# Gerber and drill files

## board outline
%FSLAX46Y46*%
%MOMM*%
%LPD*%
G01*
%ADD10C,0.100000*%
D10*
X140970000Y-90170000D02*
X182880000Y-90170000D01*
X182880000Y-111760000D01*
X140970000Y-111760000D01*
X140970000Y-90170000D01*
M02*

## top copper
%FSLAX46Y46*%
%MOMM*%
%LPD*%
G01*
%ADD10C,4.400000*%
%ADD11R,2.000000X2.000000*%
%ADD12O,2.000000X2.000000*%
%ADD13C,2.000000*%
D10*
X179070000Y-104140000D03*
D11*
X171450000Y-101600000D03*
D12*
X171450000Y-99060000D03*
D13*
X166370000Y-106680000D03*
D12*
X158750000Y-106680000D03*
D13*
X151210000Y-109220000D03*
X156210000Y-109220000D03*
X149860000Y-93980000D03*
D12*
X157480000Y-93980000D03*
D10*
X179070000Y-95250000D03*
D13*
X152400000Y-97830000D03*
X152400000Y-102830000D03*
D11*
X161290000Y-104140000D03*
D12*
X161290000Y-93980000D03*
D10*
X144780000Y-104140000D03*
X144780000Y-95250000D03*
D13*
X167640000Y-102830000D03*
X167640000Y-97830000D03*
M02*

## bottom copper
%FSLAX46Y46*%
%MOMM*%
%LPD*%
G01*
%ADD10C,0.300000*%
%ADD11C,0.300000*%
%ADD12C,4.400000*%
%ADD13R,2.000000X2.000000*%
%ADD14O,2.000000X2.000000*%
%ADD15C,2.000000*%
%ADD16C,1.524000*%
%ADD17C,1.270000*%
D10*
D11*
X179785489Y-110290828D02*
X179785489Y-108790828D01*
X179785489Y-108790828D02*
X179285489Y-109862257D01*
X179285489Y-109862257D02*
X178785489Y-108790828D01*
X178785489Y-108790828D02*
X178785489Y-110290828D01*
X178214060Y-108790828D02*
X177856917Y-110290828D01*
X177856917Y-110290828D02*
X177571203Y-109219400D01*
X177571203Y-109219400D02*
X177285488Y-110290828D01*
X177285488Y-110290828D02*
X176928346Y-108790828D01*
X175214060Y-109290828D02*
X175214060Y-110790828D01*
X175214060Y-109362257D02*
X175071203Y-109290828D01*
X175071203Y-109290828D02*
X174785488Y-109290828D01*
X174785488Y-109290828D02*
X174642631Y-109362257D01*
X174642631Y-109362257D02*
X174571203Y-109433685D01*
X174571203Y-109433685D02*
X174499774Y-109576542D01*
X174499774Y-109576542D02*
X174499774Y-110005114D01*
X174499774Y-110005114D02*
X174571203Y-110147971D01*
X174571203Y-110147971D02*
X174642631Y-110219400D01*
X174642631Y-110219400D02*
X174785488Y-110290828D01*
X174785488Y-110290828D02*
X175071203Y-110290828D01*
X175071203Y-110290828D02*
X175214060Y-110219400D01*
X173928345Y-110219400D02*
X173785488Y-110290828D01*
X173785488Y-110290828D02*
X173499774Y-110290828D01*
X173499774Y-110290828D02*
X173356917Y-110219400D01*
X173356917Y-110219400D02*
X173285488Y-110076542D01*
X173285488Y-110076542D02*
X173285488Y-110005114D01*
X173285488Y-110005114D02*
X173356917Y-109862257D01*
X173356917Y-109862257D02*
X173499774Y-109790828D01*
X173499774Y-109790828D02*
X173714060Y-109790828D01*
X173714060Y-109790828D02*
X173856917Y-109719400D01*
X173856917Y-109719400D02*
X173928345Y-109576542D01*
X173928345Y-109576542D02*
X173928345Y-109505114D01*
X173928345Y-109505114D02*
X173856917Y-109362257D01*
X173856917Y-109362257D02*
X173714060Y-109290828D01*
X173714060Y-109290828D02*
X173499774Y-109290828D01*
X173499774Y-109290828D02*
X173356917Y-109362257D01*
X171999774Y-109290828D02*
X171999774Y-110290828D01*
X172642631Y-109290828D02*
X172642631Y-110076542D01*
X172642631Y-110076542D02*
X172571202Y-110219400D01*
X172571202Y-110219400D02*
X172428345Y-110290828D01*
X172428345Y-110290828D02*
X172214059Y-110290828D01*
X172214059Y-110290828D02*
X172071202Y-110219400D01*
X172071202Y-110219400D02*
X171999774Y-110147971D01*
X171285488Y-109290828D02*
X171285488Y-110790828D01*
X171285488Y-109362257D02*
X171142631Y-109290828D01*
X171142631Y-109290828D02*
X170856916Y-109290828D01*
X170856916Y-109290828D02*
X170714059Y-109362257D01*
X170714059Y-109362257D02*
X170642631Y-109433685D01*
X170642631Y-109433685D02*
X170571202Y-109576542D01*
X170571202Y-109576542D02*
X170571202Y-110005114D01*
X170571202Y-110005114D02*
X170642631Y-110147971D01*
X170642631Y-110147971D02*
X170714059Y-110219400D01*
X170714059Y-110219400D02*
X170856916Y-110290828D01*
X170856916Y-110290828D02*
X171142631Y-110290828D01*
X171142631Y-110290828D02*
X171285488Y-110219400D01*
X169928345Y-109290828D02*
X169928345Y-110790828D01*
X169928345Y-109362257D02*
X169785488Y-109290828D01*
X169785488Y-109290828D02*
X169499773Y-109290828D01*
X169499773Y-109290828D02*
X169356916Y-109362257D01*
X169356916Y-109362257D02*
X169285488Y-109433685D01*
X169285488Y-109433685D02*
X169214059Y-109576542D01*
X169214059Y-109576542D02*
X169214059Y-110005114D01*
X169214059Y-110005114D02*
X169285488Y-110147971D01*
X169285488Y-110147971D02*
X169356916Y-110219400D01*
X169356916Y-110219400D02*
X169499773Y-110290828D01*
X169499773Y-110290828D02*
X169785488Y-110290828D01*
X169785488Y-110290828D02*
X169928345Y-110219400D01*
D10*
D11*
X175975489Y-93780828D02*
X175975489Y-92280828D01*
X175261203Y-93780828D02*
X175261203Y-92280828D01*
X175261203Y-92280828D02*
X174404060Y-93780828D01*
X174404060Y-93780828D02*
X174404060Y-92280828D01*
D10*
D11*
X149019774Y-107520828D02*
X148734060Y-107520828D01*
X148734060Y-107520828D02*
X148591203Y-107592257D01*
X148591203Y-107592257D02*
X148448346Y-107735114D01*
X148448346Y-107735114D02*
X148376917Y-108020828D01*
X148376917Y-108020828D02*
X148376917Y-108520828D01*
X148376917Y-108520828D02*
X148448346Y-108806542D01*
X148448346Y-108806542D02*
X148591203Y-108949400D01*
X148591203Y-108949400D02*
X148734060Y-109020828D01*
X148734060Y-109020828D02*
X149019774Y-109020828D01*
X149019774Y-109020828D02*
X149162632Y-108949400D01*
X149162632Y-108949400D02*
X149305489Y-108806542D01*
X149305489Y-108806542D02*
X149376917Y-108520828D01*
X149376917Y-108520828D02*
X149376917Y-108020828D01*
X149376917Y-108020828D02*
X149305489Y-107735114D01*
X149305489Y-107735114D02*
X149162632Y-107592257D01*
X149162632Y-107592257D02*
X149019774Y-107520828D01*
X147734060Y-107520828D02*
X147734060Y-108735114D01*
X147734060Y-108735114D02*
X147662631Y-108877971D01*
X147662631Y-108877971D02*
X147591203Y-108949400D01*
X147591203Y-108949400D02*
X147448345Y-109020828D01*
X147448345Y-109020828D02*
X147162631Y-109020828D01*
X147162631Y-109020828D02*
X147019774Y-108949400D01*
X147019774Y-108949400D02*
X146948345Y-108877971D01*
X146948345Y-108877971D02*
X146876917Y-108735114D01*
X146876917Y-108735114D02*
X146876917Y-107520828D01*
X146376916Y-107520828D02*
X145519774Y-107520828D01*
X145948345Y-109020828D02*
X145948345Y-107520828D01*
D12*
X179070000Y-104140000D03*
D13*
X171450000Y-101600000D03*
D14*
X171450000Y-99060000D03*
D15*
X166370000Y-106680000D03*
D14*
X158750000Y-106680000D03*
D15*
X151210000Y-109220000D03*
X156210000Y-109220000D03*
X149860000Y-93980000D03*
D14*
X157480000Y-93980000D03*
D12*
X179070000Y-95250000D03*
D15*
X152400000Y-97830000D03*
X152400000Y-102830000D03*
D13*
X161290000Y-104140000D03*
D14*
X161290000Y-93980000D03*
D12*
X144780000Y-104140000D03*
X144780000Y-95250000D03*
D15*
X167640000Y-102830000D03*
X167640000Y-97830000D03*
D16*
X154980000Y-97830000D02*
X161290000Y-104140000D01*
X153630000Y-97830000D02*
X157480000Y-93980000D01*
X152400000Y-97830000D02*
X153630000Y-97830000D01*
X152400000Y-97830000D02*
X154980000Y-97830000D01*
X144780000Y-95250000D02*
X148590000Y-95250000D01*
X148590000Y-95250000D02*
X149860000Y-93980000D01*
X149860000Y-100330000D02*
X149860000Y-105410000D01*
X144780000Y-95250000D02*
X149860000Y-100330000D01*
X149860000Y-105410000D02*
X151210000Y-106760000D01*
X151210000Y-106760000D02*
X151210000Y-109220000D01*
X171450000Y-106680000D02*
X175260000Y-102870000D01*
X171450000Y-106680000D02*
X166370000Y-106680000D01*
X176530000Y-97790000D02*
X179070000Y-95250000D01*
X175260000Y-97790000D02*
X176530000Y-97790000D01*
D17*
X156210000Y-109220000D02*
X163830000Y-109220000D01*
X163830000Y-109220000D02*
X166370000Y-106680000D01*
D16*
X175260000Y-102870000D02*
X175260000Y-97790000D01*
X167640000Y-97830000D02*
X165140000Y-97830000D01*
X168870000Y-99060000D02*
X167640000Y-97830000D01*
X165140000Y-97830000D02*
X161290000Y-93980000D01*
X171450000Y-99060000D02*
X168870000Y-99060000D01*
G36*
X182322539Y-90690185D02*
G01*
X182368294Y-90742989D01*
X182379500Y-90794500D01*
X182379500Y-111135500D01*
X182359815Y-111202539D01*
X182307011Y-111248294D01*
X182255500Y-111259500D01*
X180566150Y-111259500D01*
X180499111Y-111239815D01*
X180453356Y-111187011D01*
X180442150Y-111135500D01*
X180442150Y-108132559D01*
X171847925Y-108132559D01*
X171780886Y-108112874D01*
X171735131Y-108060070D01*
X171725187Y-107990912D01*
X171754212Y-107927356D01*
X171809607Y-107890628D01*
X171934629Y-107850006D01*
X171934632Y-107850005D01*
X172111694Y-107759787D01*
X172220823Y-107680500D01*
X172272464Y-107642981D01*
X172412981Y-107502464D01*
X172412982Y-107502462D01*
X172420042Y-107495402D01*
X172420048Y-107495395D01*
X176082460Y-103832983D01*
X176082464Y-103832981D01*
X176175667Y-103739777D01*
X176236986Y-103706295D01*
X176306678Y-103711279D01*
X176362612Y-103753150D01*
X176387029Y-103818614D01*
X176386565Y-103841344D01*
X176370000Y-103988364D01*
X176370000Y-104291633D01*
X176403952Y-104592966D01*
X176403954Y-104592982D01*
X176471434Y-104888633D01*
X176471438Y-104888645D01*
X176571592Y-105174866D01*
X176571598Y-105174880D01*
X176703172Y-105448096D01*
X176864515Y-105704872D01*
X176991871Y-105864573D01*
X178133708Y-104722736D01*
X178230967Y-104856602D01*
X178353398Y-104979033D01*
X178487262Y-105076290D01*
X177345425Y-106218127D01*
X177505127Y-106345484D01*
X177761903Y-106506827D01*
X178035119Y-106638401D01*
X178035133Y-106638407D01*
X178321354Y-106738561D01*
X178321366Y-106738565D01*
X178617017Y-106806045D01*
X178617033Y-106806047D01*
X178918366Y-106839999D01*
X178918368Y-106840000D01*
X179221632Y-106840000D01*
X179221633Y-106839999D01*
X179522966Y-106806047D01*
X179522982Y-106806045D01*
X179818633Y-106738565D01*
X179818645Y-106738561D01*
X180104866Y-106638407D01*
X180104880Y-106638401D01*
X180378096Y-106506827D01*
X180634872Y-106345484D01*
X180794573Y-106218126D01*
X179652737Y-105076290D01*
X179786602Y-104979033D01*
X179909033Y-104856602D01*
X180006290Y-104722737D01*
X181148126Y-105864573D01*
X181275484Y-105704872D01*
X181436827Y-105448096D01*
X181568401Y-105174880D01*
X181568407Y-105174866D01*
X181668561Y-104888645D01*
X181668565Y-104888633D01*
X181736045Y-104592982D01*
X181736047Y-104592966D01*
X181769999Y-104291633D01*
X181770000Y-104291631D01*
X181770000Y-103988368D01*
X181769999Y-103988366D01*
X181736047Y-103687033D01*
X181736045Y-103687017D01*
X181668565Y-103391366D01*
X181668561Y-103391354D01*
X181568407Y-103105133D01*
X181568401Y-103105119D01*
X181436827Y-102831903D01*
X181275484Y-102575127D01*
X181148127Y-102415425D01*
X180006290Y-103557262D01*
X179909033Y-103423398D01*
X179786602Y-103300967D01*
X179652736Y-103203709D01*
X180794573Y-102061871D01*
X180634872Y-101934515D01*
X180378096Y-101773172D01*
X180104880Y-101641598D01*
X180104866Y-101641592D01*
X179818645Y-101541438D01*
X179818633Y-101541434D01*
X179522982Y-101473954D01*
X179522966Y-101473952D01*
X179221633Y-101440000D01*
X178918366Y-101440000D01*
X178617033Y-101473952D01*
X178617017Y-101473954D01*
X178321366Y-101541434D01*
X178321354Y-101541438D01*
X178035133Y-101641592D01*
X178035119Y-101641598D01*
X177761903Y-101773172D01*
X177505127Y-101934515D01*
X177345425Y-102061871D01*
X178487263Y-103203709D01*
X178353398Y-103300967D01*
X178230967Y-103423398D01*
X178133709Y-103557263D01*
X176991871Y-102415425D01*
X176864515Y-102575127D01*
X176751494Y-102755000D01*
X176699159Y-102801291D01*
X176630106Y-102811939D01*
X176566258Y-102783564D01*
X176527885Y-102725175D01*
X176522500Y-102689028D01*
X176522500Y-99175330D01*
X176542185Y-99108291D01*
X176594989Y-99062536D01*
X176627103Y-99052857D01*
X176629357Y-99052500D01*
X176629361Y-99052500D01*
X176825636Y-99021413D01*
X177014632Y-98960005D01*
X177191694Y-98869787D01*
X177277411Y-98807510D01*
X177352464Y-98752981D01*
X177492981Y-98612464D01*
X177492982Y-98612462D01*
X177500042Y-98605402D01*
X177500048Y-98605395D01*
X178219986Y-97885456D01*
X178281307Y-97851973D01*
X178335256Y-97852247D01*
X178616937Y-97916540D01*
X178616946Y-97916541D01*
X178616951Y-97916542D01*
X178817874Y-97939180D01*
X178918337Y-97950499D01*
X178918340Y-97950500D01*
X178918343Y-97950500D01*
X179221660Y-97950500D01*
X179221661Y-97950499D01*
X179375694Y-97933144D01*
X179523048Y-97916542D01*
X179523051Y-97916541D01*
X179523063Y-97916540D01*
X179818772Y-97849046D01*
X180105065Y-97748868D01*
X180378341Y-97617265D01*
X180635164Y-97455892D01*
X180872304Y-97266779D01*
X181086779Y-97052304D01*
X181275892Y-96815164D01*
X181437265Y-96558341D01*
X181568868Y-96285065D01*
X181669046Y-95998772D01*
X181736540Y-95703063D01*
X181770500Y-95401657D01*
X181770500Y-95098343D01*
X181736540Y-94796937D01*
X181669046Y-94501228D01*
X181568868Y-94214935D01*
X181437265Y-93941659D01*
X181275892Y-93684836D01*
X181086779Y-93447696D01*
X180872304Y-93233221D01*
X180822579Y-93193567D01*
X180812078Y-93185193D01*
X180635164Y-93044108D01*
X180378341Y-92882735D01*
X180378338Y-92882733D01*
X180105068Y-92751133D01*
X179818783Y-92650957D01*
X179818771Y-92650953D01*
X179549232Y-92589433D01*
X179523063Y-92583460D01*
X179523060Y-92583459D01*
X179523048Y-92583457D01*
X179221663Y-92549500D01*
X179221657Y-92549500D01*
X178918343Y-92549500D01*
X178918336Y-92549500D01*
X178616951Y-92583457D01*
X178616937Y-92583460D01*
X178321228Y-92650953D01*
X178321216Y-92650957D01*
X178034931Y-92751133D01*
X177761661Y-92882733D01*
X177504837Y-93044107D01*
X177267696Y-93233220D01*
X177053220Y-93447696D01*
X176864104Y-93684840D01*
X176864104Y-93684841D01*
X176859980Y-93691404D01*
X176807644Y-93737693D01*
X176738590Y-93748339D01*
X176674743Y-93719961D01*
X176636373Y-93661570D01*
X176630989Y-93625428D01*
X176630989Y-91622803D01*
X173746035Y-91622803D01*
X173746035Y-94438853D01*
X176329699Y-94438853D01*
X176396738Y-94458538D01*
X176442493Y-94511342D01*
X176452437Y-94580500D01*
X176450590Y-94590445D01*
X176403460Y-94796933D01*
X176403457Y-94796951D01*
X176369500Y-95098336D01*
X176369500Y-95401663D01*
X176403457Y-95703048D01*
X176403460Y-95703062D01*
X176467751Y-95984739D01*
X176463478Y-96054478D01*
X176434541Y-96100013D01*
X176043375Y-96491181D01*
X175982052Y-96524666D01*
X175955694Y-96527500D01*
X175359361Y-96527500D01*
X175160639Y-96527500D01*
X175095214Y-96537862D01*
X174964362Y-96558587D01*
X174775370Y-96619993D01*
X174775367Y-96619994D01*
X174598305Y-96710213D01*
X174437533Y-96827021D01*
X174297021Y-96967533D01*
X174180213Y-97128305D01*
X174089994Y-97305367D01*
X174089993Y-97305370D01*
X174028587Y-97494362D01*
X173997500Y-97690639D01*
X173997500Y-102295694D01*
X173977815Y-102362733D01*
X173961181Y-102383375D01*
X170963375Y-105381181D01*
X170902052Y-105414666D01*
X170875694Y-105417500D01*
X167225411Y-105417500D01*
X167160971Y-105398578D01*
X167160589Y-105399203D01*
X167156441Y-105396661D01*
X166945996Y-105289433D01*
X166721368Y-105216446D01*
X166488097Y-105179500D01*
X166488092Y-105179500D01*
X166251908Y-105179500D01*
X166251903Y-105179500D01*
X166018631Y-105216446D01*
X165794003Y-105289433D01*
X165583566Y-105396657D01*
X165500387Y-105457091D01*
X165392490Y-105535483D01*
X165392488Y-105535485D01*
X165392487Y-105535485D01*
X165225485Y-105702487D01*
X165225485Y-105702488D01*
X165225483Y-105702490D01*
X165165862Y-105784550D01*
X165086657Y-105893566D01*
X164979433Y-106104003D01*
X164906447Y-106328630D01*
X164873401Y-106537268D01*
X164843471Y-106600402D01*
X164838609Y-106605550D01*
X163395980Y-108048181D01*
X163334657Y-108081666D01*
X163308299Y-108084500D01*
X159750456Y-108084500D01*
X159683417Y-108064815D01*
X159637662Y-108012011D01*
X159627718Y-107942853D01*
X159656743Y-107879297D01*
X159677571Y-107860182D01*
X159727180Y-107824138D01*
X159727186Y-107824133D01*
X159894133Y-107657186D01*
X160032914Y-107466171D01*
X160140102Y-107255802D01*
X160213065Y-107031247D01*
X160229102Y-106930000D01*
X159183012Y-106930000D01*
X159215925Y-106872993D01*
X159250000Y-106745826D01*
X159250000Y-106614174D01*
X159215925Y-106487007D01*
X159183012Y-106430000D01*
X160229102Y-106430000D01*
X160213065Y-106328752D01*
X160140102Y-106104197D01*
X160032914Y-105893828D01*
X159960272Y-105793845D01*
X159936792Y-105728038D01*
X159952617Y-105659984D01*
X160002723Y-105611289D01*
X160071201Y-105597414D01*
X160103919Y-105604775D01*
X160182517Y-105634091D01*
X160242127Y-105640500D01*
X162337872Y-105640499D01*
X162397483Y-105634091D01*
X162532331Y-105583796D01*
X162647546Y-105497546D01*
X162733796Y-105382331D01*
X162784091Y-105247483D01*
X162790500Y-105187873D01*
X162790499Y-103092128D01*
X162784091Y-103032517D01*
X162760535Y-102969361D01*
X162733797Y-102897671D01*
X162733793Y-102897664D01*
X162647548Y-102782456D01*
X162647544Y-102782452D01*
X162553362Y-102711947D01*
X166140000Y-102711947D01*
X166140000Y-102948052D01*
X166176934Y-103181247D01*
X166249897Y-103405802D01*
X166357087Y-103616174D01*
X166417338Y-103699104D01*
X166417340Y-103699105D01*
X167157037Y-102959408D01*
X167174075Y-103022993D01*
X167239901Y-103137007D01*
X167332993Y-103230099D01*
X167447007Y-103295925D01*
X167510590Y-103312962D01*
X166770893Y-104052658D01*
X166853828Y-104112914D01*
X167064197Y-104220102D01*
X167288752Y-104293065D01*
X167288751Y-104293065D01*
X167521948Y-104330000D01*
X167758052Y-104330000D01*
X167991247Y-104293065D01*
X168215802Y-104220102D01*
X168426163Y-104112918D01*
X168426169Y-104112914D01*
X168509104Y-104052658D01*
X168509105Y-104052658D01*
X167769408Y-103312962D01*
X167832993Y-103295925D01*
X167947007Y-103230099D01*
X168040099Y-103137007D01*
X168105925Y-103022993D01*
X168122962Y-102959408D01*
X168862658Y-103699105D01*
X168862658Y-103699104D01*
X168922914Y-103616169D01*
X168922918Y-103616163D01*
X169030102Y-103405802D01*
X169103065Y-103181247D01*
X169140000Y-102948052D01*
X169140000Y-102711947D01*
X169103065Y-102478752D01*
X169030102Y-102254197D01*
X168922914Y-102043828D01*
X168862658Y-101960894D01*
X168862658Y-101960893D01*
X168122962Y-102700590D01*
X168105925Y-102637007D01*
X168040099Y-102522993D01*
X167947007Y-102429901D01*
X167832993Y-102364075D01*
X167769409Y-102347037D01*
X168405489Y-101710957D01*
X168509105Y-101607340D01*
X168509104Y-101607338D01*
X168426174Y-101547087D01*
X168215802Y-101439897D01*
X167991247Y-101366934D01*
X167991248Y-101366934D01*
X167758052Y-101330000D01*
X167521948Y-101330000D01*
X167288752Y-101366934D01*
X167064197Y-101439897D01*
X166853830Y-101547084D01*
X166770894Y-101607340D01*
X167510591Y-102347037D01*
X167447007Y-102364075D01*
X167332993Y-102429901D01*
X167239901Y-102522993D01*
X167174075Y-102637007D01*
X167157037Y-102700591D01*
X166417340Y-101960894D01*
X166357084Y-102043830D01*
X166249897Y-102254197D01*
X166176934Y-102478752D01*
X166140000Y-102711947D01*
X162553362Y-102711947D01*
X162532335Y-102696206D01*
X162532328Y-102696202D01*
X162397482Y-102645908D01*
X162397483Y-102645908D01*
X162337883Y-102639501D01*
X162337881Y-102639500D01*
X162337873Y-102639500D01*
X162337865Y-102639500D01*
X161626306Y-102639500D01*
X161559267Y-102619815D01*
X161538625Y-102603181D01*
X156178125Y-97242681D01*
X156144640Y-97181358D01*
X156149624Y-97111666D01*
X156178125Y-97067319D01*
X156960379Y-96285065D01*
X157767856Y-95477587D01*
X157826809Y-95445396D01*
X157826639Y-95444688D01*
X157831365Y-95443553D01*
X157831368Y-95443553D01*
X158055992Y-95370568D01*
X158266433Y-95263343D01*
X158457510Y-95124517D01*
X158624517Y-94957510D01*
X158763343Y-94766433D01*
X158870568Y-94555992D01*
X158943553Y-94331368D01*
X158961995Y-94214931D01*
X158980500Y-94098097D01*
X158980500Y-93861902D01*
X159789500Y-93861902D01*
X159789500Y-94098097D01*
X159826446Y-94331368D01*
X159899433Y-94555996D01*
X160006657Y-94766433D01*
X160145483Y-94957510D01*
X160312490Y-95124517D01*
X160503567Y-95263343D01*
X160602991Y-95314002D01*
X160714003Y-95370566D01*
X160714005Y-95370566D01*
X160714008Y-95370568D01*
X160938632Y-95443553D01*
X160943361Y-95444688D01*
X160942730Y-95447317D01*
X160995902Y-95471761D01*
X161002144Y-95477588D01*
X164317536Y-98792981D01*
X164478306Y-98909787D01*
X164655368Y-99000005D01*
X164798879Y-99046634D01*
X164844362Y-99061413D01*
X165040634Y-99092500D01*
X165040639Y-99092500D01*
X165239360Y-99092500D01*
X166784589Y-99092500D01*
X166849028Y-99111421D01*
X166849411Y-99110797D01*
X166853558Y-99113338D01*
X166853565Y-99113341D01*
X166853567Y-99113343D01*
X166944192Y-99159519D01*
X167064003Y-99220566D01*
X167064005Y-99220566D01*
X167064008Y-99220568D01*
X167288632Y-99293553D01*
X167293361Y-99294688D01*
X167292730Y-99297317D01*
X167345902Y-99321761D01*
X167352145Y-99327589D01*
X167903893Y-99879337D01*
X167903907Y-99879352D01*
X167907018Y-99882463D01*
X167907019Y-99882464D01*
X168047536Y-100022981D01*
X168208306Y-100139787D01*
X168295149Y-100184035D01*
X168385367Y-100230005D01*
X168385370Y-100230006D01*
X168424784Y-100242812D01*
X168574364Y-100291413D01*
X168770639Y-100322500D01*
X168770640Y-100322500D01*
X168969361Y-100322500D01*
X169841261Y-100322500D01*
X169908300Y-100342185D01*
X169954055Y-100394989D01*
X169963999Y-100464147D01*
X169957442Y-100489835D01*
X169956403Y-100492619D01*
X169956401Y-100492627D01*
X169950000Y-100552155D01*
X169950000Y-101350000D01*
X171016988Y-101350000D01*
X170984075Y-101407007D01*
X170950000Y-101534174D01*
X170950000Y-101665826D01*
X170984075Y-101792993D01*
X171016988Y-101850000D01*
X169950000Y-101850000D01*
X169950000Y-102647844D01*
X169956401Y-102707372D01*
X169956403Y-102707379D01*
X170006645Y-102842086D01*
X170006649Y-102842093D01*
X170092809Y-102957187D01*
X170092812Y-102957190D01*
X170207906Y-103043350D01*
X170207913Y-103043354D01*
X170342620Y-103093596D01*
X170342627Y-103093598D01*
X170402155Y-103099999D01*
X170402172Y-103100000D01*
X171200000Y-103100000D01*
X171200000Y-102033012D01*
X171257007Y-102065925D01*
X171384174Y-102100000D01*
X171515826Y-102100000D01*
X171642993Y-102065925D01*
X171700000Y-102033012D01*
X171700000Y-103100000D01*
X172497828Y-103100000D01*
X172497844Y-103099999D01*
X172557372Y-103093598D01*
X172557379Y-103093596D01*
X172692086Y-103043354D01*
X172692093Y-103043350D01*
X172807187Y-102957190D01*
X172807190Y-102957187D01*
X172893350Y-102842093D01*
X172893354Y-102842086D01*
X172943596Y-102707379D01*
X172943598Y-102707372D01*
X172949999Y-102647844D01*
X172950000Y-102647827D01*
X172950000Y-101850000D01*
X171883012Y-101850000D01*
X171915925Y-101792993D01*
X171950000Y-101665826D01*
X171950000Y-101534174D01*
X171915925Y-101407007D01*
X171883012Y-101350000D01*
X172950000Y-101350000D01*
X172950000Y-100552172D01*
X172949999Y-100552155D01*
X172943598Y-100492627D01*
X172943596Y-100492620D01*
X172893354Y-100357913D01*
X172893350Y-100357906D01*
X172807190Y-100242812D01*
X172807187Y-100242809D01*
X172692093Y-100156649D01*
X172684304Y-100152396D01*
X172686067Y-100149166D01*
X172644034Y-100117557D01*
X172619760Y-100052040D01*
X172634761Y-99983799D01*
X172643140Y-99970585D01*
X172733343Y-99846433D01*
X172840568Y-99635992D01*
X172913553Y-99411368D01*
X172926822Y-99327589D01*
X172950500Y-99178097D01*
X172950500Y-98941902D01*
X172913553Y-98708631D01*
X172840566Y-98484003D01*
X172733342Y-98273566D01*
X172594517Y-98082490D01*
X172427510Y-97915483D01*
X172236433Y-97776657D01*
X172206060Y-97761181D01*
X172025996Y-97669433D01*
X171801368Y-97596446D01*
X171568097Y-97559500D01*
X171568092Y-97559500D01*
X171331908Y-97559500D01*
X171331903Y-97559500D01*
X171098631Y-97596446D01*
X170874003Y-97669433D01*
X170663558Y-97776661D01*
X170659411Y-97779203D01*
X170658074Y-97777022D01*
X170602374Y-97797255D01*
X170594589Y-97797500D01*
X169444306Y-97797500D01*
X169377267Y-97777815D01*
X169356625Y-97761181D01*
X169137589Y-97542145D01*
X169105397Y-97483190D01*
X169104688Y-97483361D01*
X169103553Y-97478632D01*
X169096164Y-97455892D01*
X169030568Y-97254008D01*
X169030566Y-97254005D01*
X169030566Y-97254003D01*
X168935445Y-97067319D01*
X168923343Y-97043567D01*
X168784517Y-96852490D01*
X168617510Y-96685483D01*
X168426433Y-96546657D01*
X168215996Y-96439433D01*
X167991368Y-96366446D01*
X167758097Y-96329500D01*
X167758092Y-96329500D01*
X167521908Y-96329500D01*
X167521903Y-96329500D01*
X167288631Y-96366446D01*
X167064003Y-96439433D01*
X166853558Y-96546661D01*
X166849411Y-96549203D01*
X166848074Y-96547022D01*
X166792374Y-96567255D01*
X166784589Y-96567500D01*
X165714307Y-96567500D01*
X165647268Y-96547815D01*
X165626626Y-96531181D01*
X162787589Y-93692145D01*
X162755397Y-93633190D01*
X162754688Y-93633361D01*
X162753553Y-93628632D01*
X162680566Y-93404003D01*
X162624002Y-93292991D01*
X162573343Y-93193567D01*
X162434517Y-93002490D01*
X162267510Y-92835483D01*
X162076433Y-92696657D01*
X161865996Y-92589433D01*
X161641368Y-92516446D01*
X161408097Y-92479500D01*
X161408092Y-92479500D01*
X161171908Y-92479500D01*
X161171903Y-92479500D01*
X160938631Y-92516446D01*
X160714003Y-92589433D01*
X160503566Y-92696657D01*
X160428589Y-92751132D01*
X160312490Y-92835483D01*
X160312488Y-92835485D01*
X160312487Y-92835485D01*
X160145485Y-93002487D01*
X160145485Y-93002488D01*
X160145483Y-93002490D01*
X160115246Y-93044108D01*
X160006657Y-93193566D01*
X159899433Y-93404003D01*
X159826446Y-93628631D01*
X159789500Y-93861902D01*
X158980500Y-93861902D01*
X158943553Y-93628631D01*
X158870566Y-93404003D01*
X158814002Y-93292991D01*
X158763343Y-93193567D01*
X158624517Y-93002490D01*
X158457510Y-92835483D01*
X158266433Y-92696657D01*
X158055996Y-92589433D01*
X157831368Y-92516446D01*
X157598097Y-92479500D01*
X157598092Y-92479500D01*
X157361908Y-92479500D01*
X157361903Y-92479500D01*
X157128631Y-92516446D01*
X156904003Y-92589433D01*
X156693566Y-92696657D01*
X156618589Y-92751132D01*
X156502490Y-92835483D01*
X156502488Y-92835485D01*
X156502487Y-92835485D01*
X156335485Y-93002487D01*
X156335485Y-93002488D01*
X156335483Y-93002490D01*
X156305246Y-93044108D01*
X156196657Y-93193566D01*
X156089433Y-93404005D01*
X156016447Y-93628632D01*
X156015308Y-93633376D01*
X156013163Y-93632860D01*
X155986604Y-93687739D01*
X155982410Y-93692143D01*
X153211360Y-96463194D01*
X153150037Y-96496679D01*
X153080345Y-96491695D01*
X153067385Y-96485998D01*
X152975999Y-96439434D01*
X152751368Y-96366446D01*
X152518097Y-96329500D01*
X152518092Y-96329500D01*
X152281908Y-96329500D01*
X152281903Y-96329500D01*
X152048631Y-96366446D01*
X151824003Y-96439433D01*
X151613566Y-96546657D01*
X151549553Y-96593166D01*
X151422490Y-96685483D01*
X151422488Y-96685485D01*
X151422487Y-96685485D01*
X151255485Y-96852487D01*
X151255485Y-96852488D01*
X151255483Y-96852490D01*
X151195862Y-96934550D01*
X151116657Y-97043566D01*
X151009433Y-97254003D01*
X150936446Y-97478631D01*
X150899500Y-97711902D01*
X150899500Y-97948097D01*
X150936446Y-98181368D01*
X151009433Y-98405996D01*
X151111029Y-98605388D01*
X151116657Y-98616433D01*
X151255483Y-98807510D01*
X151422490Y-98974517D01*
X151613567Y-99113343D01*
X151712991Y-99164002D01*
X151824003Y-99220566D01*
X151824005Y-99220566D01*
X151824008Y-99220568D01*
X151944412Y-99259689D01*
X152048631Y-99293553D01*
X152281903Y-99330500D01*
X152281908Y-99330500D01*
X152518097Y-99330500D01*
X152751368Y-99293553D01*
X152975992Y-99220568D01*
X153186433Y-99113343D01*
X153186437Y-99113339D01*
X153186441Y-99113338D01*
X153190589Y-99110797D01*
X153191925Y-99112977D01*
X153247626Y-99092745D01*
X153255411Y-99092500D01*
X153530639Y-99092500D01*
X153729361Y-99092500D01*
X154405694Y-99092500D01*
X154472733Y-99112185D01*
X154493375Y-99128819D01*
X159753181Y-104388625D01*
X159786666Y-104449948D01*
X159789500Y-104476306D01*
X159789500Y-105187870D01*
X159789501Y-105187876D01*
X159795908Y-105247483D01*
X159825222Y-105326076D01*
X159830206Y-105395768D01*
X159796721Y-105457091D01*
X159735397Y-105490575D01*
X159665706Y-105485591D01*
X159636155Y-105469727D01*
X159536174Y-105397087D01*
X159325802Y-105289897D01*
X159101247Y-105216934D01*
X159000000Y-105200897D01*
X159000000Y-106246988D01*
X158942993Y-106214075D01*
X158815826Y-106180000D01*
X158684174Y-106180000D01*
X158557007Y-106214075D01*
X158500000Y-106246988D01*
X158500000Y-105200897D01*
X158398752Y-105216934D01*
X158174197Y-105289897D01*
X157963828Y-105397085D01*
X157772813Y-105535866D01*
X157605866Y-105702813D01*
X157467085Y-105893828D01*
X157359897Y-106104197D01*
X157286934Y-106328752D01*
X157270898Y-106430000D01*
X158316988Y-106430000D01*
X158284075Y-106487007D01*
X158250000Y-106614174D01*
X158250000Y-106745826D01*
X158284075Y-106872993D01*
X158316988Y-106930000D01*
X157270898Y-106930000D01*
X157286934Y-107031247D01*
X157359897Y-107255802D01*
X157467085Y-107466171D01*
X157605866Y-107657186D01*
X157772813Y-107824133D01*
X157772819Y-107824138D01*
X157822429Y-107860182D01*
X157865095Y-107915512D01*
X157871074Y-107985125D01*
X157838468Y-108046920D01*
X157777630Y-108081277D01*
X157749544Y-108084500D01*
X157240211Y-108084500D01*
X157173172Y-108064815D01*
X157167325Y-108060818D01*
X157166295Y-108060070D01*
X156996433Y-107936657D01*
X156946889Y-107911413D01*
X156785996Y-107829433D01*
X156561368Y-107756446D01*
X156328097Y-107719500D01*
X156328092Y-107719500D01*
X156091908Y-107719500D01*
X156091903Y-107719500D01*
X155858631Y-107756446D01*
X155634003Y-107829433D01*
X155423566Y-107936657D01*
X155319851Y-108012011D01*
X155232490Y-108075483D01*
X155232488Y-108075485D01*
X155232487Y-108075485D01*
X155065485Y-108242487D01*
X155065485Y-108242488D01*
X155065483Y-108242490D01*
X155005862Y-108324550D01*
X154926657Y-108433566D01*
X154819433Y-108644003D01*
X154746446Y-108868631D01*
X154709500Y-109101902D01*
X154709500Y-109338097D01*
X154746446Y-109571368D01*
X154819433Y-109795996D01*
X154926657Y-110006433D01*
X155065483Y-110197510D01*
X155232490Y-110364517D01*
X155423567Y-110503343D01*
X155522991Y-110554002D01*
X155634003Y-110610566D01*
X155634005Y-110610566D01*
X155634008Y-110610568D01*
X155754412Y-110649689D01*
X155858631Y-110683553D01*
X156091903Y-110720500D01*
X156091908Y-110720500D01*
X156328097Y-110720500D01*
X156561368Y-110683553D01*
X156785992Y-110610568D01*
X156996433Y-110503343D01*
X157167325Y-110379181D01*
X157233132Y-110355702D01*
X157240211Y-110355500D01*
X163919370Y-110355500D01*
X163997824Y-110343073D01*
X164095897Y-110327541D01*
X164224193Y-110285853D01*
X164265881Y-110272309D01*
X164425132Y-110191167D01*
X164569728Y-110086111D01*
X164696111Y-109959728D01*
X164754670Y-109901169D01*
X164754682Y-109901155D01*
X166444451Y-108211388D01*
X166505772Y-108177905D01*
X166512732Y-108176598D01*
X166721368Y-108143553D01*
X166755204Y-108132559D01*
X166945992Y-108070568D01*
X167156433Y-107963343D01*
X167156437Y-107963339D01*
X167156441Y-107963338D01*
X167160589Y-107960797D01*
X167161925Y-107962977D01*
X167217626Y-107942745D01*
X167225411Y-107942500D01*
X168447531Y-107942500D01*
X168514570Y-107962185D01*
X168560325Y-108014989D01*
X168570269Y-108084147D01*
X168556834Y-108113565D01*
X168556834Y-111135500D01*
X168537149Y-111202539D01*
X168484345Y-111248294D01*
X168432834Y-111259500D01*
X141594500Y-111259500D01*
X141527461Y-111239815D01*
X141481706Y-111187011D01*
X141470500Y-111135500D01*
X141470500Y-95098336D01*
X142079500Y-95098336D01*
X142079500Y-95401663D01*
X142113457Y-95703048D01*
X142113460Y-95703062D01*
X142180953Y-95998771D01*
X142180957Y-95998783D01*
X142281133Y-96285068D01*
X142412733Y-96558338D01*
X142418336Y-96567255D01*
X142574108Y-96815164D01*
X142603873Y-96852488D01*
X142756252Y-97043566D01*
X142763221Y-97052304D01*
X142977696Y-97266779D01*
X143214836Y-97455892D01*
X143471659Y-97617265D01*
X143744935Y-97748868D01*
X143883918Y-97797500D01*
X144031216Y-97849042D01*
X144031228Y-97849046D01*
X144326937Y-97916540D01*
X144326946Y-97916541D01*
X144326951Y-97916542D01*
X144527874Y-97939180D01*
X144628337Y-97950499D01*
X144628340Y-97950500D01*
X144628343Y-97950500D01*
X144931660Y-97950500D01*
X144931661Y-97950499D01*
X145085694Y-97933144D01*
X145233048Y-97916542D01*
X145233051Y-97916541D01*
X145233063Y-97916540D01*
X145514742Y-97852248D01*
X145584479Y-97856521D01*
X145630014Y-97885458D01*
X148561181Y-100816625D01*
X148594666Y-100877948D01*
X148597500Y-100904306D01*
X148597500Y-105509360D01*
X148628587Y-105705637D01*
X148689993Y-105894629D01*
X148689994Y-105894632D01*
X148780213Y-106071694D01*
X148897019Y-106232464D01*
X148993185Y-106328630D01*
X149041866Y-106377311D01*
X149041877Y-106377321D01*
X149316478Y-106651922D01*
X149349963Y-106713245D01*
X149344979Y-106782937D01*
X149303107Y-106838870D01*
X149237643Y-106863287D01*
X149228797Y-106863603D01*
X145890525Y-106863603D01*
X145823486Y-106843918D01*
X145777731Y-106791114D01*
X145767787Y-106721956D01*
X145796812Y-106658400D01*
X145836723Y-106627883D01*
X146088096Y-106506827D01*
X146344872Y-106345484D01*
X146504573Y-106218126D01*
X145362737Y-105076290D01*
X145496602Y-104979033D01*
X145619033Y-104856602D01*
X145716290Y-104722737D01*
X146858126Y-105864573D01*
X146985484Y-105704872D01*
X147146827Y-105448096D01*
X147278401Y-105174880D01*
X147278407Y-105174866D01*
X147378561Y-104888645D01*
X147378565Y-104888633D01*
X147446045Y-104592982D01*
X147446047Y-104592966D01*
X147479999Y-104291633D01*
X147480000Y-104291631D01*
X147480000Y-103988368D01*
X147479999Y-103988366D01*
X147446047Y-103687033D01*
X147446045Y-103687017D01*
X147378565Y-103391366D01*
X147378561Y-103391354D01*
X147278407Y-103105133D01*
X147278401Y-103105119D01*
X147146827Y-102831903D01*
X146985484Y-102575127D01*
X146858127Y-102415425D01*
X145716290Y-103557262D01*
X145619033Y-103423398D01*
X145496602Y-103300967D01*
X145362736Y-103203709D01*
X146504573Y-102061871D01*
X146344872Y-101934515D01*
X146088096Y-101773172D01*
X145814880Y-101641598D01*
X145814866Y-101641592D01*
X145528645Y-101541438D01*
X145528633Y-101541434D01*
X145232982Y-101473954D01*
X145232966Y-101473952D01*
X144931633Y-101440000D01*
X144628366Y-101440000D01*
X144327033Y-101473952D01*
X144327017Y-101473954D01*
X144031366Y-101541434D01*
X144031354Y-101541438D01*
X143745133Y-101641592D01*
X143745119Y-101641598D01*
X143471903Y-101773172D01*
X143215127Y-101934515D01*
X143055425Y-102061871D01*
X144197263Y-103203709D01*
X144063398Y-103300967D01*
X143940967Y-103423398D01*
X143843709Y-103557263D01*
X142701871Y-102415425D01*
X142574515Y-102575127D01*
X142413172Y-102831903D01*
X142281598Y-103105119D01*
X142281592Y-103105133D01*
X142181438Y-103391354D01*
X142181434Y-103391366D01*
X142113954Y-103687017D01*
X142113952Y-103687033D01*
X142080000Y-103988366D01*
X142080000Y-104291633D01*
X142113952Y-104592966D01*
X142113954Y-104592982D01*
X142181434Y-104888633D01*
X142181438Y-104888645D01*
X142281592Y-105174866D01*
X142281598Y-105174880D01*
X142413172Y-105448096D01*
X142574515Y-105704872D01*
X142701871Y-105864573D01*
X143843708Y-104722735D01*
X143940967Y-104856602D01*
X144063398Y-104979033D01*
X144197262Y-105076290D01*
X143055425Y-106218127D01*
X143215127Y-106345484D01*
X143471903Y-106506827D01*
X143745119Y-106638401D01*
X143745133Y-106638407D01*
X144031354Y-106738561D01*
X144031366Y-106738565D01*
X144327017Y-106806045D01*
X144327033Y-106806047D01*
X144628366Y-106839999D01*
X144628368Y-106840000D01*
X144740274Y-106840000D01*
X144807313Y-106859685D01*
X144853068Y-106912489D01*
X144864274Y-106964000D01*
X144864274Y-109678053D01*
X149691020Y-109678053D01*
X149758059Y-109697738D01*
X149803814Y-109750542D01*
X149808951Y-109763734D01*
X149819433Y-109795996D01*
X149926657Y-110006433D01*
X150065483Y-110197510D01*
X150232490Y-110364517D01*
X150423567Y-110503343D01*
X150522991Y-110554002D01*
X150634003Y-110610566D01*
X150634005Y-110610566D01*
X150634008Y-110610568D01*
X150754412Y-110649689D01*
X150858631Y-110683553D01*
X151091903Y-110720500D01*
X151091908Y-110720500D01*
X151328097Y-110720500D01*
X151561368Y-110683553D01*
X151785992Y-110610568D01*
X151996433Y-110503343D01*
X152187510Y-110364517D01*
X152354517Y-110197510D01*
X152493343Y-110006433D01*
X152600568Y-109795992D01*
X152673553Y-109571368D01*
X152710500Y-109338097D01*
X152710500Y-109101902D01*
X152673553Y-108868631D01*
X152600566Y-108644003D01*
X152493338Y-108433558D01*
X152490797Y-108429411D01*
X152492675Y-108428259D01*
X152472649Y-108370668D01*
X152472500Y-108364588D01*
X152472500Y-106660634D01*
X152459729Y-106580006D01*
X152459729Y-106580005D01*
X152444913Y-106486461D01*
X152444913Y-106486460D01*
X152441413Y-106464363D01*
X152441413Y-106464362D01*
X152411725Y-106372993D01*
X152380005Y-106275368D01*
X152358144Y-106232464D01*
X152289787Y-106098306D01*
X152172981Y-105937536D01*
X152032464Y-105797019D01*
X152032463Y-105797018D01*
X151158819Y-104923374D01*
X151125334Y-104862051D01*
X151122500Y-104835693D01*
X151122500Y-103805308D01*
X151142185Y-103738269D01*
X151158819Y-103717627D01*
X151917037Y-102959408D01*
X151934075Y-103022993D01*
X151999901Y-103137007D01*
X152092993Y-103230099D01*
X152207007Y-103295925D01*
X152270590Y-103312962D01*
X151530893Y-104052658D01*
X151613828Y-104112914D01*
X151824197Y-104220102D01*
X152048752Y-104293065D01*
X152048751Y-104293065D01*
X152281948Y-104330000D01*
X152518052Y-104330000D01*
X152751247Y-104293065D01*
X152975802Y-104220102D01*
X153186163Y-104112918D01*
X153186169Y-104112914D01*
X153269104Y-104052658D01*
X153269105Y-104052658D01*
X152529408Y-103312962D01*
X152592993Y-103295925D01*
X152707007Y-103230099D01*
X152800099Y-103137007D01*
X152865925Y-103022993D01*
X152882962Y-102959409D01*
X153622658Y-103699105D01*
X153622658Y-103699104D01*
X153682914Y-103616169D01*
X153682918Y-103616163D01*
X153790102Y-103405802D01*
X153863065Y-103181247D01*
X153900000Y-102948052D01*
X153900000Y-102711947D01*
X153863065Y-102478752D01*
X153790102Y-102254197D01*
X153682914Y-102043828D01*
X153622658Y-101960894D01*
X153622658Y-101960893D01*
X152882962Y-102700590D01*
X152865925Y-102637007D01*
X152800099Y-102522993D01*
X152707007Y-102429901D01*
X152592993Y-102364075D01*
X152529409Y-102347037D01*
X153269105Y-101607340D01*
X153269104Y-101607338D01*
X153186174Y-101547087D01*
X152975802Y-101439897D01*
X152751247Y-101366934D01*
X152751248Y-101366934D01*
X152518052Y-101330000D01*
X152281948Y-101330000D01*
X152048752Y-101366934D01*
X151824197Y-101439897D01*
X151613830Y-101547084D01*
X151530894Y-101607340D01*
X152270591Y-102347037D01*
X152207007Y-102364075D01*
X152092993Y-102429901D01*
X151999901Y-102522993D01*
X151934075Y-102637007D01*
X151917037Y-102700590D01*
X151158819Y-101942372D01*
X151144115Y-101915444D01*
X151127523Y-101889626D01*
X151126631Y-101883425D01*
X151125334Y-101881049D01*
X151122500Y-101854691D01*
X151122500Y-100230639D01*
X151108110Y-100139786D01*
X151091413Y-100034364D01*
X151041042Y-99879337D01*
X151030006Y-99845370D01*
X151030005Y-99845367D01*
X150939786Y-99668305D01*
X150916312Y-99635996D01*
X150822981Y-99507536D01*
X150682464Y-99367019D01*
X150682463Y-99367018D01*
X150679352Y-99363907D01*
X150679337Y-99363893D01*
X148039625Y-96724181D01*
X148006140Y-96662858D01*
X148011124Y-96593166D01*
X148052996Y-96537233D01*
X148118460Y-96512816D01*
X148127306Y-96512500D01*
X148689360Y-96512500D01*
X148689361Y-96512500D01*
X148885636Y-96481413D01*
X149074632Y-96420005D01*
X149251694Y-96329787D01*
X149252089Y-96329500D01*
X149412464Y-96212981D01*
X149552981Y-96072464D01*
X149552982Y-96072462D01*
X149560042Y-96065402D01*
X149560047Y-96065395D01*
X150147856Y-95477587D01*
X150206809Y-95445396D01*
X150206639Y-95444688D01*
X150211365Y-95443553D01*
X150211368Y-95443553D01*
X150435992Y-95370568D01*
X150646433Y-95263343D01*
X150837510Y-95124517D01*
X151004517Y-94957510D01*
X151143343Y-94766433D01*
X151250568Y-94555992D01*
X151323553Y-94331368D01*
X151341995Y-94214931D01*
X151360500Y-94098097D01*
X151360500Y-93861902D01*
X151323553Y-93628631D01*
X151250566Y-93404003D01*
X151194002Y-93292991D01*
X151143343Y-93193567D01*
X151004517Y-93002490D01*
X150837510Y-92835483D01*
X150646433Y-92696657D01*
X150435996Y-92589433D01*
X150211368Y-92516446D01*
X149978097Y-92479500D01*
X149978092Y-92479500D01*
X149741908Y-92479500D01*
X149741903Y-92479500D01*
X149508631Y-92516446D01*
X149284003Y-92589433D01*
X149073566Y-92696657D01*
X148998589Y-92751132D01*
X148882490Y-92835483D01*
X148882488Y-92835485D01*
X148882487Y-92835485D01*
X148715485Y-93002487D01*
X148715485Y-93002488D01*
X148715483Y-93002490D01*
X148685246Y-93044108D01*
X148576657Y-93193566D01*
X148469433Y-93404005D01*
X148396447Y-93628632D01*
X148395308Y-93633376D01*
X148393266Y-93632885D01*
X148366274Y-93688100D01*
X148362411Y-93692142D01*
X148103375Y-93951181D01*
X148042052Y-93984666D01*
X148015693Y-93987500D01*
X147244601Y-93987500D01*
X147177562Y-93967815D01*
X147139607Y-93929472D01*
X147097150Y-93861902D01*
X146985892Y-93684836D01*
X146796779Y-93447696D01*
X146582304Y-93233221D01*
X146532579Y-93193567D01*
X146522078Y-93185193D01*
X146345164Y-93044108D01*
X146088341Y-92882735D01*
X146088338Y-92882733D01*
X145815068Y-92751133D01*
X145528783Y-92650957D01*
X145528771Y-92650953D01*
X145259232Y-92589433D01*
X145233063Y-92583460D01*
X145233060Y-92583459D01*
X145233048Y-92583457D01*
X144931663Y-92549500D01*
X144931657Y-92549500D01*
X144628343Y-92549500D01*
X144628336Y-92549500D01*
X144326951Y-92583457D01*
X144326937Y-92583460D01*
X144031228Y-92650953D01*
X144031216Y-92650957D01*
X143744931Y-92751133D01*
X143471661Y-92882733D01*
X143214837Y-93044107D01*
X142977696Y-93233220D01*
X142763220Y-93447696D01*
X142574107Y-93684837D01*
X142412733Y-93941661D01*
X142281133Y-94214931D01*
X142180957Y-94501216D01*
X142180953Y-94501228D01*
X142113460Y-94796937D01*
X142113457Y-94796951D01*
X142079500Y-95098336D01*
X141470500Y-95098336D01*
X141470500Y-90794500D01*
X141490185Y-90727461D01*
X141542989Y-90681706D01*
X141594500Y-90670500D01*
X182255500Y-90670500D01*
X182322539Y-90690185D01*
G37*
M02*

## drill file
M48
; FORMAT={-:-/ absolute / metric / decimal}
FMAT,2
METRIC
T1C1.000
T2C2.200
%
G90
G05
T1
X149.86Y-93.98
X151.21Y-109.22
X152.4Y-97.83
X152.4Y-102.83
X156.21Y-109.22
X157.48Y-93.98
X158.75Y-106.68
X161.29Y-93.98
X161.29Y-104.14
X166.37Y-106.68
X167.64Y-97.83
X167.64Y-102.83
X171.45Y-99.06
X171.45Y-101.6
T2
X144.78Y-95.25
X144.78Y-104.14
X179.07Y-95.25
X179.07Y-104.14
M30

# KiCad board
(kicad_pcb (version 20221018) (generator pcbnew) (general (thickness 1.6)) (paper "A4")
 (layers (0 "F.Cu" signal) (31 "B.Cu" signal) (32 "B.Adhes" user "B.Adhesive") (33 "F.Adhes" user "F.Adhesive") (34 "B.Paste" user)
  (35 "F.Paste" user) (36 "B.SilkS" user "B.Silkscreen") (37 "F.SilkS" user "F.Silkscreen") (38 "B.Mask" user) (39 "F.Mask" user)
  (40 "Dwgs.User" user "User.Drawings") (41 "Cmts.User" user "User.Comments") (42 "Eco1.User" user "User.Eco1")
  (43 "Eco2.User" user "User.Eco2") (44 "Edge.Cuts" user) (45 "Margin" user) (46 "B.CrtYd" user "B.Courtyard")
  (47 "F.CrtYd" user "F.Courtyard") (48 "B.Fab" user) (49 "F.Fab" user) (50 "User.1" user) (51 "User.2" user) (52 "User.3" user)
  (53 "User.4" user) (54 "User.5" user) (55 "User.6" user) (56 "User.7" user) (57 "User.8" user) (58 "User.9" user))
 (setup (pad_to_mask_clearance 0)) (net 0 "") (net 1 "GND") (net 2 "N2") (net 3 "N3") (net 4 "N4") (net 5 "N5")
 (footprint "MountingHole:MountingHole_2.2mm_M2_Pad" (layer "F.Cu") (at 179.07 104.14)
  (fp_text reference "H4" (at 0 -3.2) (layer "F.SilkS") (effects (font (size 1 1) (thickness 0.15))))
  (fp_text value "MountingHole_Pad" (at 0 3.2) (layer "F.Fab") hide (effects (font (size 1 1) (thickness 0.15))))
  (pad "1" thru_hole circle (at 0 0) (size 4.4 4.4) (drill 2.2) (layers "*.Cu" "*.Mask") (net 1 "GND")))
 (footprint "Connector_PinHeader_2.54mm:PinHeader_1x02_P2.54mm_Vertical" (layer "F.Cu") (at 171.45 101.6 180)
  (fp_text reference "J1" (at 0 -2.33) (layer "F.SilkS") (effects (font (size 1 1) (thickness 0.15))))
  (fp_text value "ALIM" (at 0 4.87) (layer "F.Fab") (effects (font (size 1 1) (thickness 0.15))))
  (pad "1" thru_hole rect (at 0 0 180) (size 2 2) (drill 1) (layers "*.Cu" "*.Mask") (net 1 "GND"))
  (pad "2" thru_hole oval (at 0 2.54 180) (size 2 2) (drill 1) (layers "*.Cu" "*.Mask") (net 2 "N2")))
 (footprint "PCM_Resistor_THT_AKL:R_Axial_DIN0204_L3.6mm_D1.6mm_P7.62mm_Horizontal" (layer "F.Cu") (at 166.37 106.68 180)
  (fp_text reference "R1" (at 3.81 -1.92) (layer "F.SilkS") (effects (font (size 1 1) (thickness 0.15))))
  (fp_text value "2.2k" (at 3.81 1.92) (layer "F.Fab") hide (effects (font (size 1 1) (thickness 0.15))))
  (pad "1" thru_hole circle (at 0 0 180) (size 2 2) (drill 1) (layers "*.Cu" "*.Mask") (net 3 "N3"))
  (pad "2" thru_hole oval (at 7.62 0 180) (size 2 2) (drill 1) (layers "*.Cu" "*.Mask") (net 1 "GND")))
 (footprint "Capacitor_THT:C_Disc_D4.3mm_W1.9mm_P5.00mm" (layer "F.Cu") (at 151.21 109.22)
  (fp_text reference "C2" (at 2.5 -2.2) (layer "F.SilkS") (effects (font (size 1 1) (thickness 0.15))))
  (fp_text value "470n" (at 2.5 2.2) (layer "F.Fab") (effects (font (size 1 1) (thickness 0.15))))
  (pad "1" thru_hole circle (at 0 0) (size 2 2) (drill 1) (layers "*.Cu" "*.Mask") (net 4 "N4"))
  (pad "2" thru_hole circle (at 5 0) (size 2 2) (drill 1) (layers "*.Cu" "*.Mask") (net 3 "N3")))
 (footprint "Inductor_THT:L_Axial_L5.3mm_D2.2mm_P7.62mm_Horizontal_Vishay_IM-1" (layer "F.Cu") (at 149.86 93.98)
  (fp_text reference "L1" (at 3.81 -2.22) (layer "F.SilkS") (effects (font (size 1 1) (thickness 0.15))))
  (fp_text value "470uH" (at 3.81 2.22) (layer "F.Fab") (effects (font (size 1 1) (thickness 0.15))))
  (pad "1" thru_hole circle (at 0 0) (size 2 2) (drill 1) (layers "*.Cu" "*.Mask") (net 4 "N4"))
  (pad "2" thru_hole oval (at 7.62 0) (size 2 2) (drill 1) (layers "*.Cu" "*.Mask") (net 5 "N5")))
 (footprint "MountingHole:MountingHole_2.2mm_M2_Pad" (layer "F.Cu") (at 179.07 95.25)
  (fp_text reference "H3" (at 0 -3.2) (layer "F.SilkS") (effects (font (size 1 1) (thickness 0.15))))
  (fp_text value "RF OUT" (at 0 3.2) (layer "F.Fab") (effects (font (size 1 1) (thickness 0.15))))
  (pad "1" thru_hole circle (at 0 0) (size 4.4 4.4) (drill 2.2) (layers "*.Cu" "*.Mask") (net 3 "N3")))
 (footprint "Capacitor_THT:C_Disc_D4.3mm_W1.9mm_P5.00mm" (layer "F.Cu") (at 152.4 97.83 -90)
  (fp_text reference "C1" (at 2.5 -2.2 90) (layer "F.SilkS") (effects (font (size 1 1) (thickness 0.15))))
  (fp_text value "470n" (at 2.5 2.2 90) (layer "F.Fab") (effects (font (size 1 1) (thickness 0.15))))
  (pad "1" thru_hole circle (at 0 0 270) (size 2 2) (drill 1) (layers "*.Cu" "*.Mask") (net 5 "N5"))
  (pad "2" thru_hole circle (at 5 0 270) (size 2 2) (drill 1) (layers "*.Cu" "*.Mask") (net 1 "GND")))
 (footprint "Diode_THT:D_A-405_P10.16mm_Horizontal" (layer "F.Cu") (at 161.29 104.14 90)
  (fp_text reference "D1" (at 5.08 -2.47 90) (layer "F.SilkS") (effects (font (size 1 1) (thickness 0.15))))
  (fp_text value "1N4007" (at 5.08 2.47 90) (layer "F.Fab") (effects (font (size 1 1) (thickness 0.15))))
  (pad "1" thru_hole rect (at 0 0 90) (size 2 2) (drill 1) (layers "*.Cu" "*.Mask") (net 5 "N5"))
  (pad "2" thru_hole oval (at 10.16 0 90) (size 2 2) (drill 1) (layers "*.Cu" "*.Mask") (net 2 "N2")))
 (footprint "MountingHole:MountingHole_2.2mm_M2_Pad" (layer "F.Cu") (at 144.78 104.14)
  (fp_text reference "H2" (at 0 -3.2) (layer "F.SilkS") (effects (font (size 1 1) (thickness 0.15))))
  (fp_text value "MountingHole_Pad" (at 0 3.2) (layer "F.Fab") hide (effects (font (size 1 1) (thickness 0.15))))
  (pad "1" thru_hole circle (at 0 0) (size 4.4 4.4) (drill 2.2) (layers "*.Cu" "*.Mask") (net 1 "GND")))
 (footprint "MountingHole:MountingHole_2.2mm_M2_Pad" (layer "F.Cu") (at 144.78 95.25)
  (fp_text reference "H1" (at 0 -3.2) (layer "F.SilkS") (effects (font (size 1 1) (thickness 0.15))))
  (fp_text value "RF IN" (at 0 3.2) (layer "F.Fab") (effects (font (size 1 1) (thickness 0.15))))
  (pad "1" thru_hole circle (at 0 0) (size 4.4 4.4) (drill 2.2) (layers "*.Cu" "*.Mask") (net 4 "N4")))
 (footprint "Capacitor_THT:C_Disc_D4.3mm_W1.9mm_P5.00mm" (layer "F.Cu") (at 167.64 102.83 90)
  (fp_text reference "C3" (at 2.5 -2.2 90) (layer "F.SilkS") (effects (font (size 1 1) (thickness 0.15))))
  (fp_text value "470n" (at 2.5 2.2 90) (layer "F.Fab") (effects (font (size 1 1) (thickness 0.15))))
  (pad "1" thru_hole circle (at 0 0 90) (size 2 2) (drill 1) (layers "*.Cu" "*.Mask") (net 1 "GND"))
  (pad "2" thru_hole circle (at 5 0 90) (size 2 2) (drill 1) (layers "*.Cu" "*.Mask") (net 2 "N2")))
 (gr_rect (start 140.97 90.17) (end 182.88 111.76) (stroke (width 0.1) (type default)) (fill none) (layer "Edge.Cuts"))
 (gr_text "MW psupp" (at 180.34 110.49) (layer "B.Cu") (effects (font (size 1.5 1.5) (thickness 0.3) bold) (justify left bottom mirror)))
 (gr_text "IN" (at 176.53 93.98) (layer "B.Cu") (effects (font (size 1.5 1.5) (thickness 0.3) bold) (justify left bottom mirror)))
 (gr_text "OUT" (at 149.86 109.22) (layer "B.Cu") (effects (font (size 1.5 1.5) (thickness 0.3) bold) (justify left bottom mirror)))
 (segment (start 154.98 97.83) (end 161.29 104.14) (width 1.524) (layer "B.Cu") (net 5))
 (segment (start 153.63 97.83) (end 157.48 93.98) (width 1.524) (layer "B.Cu") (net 5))
 (segment (start 152.4 97.83) (end 153.63 97.83) (width 1.524) (layer "B.Cu") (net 5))
 (segment (start 152.4 97.83) (end 154.98 97.83) (width 1.524) (layer "B.Cu") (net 5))
 (segment (start 144.78 95.25) (end 148.59 95.25) (width 1.524) (layer "B.Cu") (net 4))
 (segment (start 148.59 95.25) (end 149.86 93.98) (width 1.524) (layer "B.Cu") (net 4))
 (segment (start 149.86 100.33) (end 149.86 105.41) (width 1.524) (layer "B.Cu") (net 4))
 (segment (start 144.78 95.25) (end 149.86 100.33) (width 1.524) (layer "B.Cu") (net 4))
 (segment (start 149.86 105.41) (end 151.21 106.76) (width 1.524) (layer "B.Cu") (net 4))
 (segment (start 151.21 106.76) (end 151.21 109.22) (width 1.524) (layer "B.Cu") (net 4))
 (segment (start 171.45 106.68) (end 175.26 102.87) (width 1.524) (layer "B.Cu") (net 3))
 (segment (start 171.45 106.68) (end 166.37 106.68) (width 1.524) (layer "B.Cu") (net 3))
 (segment (start 176.53 97.79) (end 179.07 95.25) (width 1.524) (layer "B.Cu") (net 3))
 (segment (start 175.26 97.79) (end 176.53 97.79) (width 1.524) (layer "B.Cu") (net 3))
 (segment (start 156.21 109.22) (end 163.83 109.22) (width 1.27) (layer "B.Cu") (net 3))
 (segment (start 163.83 109.22) (end 166.37 106.68) (width 1.27) (layer "B.Cu") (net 3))
 (segment (start 175.26 102.87) (end 175.26 97.79) (width 1.524) (layer "B.Cu") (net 3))
 (segment (start 167.64 97.83) (end 165.14 97.83) (width 1.524) (layer "B.Cu") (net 2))
 (segment (start 168.87 99.06) (end 167.64 97.83) (width 1.524) (layer "B.Cu") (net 2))
 (segment (start 165.14 97.83) (end 161.29 93.98) (width 1.524) (layer "B.Cu") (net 2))
 (segment (start 171.45 99.06) (end 168.87 99.06) (width 1.524) (layer "B.Cu") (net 2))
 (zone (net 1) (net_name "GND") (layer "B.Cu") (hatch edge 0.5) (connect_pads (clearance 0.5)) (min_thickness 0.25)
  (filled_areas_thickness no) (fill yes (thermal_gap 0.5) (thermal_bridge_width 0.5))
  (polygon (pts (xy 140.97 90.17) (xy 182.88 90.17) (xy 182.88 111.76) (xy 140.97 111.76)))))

